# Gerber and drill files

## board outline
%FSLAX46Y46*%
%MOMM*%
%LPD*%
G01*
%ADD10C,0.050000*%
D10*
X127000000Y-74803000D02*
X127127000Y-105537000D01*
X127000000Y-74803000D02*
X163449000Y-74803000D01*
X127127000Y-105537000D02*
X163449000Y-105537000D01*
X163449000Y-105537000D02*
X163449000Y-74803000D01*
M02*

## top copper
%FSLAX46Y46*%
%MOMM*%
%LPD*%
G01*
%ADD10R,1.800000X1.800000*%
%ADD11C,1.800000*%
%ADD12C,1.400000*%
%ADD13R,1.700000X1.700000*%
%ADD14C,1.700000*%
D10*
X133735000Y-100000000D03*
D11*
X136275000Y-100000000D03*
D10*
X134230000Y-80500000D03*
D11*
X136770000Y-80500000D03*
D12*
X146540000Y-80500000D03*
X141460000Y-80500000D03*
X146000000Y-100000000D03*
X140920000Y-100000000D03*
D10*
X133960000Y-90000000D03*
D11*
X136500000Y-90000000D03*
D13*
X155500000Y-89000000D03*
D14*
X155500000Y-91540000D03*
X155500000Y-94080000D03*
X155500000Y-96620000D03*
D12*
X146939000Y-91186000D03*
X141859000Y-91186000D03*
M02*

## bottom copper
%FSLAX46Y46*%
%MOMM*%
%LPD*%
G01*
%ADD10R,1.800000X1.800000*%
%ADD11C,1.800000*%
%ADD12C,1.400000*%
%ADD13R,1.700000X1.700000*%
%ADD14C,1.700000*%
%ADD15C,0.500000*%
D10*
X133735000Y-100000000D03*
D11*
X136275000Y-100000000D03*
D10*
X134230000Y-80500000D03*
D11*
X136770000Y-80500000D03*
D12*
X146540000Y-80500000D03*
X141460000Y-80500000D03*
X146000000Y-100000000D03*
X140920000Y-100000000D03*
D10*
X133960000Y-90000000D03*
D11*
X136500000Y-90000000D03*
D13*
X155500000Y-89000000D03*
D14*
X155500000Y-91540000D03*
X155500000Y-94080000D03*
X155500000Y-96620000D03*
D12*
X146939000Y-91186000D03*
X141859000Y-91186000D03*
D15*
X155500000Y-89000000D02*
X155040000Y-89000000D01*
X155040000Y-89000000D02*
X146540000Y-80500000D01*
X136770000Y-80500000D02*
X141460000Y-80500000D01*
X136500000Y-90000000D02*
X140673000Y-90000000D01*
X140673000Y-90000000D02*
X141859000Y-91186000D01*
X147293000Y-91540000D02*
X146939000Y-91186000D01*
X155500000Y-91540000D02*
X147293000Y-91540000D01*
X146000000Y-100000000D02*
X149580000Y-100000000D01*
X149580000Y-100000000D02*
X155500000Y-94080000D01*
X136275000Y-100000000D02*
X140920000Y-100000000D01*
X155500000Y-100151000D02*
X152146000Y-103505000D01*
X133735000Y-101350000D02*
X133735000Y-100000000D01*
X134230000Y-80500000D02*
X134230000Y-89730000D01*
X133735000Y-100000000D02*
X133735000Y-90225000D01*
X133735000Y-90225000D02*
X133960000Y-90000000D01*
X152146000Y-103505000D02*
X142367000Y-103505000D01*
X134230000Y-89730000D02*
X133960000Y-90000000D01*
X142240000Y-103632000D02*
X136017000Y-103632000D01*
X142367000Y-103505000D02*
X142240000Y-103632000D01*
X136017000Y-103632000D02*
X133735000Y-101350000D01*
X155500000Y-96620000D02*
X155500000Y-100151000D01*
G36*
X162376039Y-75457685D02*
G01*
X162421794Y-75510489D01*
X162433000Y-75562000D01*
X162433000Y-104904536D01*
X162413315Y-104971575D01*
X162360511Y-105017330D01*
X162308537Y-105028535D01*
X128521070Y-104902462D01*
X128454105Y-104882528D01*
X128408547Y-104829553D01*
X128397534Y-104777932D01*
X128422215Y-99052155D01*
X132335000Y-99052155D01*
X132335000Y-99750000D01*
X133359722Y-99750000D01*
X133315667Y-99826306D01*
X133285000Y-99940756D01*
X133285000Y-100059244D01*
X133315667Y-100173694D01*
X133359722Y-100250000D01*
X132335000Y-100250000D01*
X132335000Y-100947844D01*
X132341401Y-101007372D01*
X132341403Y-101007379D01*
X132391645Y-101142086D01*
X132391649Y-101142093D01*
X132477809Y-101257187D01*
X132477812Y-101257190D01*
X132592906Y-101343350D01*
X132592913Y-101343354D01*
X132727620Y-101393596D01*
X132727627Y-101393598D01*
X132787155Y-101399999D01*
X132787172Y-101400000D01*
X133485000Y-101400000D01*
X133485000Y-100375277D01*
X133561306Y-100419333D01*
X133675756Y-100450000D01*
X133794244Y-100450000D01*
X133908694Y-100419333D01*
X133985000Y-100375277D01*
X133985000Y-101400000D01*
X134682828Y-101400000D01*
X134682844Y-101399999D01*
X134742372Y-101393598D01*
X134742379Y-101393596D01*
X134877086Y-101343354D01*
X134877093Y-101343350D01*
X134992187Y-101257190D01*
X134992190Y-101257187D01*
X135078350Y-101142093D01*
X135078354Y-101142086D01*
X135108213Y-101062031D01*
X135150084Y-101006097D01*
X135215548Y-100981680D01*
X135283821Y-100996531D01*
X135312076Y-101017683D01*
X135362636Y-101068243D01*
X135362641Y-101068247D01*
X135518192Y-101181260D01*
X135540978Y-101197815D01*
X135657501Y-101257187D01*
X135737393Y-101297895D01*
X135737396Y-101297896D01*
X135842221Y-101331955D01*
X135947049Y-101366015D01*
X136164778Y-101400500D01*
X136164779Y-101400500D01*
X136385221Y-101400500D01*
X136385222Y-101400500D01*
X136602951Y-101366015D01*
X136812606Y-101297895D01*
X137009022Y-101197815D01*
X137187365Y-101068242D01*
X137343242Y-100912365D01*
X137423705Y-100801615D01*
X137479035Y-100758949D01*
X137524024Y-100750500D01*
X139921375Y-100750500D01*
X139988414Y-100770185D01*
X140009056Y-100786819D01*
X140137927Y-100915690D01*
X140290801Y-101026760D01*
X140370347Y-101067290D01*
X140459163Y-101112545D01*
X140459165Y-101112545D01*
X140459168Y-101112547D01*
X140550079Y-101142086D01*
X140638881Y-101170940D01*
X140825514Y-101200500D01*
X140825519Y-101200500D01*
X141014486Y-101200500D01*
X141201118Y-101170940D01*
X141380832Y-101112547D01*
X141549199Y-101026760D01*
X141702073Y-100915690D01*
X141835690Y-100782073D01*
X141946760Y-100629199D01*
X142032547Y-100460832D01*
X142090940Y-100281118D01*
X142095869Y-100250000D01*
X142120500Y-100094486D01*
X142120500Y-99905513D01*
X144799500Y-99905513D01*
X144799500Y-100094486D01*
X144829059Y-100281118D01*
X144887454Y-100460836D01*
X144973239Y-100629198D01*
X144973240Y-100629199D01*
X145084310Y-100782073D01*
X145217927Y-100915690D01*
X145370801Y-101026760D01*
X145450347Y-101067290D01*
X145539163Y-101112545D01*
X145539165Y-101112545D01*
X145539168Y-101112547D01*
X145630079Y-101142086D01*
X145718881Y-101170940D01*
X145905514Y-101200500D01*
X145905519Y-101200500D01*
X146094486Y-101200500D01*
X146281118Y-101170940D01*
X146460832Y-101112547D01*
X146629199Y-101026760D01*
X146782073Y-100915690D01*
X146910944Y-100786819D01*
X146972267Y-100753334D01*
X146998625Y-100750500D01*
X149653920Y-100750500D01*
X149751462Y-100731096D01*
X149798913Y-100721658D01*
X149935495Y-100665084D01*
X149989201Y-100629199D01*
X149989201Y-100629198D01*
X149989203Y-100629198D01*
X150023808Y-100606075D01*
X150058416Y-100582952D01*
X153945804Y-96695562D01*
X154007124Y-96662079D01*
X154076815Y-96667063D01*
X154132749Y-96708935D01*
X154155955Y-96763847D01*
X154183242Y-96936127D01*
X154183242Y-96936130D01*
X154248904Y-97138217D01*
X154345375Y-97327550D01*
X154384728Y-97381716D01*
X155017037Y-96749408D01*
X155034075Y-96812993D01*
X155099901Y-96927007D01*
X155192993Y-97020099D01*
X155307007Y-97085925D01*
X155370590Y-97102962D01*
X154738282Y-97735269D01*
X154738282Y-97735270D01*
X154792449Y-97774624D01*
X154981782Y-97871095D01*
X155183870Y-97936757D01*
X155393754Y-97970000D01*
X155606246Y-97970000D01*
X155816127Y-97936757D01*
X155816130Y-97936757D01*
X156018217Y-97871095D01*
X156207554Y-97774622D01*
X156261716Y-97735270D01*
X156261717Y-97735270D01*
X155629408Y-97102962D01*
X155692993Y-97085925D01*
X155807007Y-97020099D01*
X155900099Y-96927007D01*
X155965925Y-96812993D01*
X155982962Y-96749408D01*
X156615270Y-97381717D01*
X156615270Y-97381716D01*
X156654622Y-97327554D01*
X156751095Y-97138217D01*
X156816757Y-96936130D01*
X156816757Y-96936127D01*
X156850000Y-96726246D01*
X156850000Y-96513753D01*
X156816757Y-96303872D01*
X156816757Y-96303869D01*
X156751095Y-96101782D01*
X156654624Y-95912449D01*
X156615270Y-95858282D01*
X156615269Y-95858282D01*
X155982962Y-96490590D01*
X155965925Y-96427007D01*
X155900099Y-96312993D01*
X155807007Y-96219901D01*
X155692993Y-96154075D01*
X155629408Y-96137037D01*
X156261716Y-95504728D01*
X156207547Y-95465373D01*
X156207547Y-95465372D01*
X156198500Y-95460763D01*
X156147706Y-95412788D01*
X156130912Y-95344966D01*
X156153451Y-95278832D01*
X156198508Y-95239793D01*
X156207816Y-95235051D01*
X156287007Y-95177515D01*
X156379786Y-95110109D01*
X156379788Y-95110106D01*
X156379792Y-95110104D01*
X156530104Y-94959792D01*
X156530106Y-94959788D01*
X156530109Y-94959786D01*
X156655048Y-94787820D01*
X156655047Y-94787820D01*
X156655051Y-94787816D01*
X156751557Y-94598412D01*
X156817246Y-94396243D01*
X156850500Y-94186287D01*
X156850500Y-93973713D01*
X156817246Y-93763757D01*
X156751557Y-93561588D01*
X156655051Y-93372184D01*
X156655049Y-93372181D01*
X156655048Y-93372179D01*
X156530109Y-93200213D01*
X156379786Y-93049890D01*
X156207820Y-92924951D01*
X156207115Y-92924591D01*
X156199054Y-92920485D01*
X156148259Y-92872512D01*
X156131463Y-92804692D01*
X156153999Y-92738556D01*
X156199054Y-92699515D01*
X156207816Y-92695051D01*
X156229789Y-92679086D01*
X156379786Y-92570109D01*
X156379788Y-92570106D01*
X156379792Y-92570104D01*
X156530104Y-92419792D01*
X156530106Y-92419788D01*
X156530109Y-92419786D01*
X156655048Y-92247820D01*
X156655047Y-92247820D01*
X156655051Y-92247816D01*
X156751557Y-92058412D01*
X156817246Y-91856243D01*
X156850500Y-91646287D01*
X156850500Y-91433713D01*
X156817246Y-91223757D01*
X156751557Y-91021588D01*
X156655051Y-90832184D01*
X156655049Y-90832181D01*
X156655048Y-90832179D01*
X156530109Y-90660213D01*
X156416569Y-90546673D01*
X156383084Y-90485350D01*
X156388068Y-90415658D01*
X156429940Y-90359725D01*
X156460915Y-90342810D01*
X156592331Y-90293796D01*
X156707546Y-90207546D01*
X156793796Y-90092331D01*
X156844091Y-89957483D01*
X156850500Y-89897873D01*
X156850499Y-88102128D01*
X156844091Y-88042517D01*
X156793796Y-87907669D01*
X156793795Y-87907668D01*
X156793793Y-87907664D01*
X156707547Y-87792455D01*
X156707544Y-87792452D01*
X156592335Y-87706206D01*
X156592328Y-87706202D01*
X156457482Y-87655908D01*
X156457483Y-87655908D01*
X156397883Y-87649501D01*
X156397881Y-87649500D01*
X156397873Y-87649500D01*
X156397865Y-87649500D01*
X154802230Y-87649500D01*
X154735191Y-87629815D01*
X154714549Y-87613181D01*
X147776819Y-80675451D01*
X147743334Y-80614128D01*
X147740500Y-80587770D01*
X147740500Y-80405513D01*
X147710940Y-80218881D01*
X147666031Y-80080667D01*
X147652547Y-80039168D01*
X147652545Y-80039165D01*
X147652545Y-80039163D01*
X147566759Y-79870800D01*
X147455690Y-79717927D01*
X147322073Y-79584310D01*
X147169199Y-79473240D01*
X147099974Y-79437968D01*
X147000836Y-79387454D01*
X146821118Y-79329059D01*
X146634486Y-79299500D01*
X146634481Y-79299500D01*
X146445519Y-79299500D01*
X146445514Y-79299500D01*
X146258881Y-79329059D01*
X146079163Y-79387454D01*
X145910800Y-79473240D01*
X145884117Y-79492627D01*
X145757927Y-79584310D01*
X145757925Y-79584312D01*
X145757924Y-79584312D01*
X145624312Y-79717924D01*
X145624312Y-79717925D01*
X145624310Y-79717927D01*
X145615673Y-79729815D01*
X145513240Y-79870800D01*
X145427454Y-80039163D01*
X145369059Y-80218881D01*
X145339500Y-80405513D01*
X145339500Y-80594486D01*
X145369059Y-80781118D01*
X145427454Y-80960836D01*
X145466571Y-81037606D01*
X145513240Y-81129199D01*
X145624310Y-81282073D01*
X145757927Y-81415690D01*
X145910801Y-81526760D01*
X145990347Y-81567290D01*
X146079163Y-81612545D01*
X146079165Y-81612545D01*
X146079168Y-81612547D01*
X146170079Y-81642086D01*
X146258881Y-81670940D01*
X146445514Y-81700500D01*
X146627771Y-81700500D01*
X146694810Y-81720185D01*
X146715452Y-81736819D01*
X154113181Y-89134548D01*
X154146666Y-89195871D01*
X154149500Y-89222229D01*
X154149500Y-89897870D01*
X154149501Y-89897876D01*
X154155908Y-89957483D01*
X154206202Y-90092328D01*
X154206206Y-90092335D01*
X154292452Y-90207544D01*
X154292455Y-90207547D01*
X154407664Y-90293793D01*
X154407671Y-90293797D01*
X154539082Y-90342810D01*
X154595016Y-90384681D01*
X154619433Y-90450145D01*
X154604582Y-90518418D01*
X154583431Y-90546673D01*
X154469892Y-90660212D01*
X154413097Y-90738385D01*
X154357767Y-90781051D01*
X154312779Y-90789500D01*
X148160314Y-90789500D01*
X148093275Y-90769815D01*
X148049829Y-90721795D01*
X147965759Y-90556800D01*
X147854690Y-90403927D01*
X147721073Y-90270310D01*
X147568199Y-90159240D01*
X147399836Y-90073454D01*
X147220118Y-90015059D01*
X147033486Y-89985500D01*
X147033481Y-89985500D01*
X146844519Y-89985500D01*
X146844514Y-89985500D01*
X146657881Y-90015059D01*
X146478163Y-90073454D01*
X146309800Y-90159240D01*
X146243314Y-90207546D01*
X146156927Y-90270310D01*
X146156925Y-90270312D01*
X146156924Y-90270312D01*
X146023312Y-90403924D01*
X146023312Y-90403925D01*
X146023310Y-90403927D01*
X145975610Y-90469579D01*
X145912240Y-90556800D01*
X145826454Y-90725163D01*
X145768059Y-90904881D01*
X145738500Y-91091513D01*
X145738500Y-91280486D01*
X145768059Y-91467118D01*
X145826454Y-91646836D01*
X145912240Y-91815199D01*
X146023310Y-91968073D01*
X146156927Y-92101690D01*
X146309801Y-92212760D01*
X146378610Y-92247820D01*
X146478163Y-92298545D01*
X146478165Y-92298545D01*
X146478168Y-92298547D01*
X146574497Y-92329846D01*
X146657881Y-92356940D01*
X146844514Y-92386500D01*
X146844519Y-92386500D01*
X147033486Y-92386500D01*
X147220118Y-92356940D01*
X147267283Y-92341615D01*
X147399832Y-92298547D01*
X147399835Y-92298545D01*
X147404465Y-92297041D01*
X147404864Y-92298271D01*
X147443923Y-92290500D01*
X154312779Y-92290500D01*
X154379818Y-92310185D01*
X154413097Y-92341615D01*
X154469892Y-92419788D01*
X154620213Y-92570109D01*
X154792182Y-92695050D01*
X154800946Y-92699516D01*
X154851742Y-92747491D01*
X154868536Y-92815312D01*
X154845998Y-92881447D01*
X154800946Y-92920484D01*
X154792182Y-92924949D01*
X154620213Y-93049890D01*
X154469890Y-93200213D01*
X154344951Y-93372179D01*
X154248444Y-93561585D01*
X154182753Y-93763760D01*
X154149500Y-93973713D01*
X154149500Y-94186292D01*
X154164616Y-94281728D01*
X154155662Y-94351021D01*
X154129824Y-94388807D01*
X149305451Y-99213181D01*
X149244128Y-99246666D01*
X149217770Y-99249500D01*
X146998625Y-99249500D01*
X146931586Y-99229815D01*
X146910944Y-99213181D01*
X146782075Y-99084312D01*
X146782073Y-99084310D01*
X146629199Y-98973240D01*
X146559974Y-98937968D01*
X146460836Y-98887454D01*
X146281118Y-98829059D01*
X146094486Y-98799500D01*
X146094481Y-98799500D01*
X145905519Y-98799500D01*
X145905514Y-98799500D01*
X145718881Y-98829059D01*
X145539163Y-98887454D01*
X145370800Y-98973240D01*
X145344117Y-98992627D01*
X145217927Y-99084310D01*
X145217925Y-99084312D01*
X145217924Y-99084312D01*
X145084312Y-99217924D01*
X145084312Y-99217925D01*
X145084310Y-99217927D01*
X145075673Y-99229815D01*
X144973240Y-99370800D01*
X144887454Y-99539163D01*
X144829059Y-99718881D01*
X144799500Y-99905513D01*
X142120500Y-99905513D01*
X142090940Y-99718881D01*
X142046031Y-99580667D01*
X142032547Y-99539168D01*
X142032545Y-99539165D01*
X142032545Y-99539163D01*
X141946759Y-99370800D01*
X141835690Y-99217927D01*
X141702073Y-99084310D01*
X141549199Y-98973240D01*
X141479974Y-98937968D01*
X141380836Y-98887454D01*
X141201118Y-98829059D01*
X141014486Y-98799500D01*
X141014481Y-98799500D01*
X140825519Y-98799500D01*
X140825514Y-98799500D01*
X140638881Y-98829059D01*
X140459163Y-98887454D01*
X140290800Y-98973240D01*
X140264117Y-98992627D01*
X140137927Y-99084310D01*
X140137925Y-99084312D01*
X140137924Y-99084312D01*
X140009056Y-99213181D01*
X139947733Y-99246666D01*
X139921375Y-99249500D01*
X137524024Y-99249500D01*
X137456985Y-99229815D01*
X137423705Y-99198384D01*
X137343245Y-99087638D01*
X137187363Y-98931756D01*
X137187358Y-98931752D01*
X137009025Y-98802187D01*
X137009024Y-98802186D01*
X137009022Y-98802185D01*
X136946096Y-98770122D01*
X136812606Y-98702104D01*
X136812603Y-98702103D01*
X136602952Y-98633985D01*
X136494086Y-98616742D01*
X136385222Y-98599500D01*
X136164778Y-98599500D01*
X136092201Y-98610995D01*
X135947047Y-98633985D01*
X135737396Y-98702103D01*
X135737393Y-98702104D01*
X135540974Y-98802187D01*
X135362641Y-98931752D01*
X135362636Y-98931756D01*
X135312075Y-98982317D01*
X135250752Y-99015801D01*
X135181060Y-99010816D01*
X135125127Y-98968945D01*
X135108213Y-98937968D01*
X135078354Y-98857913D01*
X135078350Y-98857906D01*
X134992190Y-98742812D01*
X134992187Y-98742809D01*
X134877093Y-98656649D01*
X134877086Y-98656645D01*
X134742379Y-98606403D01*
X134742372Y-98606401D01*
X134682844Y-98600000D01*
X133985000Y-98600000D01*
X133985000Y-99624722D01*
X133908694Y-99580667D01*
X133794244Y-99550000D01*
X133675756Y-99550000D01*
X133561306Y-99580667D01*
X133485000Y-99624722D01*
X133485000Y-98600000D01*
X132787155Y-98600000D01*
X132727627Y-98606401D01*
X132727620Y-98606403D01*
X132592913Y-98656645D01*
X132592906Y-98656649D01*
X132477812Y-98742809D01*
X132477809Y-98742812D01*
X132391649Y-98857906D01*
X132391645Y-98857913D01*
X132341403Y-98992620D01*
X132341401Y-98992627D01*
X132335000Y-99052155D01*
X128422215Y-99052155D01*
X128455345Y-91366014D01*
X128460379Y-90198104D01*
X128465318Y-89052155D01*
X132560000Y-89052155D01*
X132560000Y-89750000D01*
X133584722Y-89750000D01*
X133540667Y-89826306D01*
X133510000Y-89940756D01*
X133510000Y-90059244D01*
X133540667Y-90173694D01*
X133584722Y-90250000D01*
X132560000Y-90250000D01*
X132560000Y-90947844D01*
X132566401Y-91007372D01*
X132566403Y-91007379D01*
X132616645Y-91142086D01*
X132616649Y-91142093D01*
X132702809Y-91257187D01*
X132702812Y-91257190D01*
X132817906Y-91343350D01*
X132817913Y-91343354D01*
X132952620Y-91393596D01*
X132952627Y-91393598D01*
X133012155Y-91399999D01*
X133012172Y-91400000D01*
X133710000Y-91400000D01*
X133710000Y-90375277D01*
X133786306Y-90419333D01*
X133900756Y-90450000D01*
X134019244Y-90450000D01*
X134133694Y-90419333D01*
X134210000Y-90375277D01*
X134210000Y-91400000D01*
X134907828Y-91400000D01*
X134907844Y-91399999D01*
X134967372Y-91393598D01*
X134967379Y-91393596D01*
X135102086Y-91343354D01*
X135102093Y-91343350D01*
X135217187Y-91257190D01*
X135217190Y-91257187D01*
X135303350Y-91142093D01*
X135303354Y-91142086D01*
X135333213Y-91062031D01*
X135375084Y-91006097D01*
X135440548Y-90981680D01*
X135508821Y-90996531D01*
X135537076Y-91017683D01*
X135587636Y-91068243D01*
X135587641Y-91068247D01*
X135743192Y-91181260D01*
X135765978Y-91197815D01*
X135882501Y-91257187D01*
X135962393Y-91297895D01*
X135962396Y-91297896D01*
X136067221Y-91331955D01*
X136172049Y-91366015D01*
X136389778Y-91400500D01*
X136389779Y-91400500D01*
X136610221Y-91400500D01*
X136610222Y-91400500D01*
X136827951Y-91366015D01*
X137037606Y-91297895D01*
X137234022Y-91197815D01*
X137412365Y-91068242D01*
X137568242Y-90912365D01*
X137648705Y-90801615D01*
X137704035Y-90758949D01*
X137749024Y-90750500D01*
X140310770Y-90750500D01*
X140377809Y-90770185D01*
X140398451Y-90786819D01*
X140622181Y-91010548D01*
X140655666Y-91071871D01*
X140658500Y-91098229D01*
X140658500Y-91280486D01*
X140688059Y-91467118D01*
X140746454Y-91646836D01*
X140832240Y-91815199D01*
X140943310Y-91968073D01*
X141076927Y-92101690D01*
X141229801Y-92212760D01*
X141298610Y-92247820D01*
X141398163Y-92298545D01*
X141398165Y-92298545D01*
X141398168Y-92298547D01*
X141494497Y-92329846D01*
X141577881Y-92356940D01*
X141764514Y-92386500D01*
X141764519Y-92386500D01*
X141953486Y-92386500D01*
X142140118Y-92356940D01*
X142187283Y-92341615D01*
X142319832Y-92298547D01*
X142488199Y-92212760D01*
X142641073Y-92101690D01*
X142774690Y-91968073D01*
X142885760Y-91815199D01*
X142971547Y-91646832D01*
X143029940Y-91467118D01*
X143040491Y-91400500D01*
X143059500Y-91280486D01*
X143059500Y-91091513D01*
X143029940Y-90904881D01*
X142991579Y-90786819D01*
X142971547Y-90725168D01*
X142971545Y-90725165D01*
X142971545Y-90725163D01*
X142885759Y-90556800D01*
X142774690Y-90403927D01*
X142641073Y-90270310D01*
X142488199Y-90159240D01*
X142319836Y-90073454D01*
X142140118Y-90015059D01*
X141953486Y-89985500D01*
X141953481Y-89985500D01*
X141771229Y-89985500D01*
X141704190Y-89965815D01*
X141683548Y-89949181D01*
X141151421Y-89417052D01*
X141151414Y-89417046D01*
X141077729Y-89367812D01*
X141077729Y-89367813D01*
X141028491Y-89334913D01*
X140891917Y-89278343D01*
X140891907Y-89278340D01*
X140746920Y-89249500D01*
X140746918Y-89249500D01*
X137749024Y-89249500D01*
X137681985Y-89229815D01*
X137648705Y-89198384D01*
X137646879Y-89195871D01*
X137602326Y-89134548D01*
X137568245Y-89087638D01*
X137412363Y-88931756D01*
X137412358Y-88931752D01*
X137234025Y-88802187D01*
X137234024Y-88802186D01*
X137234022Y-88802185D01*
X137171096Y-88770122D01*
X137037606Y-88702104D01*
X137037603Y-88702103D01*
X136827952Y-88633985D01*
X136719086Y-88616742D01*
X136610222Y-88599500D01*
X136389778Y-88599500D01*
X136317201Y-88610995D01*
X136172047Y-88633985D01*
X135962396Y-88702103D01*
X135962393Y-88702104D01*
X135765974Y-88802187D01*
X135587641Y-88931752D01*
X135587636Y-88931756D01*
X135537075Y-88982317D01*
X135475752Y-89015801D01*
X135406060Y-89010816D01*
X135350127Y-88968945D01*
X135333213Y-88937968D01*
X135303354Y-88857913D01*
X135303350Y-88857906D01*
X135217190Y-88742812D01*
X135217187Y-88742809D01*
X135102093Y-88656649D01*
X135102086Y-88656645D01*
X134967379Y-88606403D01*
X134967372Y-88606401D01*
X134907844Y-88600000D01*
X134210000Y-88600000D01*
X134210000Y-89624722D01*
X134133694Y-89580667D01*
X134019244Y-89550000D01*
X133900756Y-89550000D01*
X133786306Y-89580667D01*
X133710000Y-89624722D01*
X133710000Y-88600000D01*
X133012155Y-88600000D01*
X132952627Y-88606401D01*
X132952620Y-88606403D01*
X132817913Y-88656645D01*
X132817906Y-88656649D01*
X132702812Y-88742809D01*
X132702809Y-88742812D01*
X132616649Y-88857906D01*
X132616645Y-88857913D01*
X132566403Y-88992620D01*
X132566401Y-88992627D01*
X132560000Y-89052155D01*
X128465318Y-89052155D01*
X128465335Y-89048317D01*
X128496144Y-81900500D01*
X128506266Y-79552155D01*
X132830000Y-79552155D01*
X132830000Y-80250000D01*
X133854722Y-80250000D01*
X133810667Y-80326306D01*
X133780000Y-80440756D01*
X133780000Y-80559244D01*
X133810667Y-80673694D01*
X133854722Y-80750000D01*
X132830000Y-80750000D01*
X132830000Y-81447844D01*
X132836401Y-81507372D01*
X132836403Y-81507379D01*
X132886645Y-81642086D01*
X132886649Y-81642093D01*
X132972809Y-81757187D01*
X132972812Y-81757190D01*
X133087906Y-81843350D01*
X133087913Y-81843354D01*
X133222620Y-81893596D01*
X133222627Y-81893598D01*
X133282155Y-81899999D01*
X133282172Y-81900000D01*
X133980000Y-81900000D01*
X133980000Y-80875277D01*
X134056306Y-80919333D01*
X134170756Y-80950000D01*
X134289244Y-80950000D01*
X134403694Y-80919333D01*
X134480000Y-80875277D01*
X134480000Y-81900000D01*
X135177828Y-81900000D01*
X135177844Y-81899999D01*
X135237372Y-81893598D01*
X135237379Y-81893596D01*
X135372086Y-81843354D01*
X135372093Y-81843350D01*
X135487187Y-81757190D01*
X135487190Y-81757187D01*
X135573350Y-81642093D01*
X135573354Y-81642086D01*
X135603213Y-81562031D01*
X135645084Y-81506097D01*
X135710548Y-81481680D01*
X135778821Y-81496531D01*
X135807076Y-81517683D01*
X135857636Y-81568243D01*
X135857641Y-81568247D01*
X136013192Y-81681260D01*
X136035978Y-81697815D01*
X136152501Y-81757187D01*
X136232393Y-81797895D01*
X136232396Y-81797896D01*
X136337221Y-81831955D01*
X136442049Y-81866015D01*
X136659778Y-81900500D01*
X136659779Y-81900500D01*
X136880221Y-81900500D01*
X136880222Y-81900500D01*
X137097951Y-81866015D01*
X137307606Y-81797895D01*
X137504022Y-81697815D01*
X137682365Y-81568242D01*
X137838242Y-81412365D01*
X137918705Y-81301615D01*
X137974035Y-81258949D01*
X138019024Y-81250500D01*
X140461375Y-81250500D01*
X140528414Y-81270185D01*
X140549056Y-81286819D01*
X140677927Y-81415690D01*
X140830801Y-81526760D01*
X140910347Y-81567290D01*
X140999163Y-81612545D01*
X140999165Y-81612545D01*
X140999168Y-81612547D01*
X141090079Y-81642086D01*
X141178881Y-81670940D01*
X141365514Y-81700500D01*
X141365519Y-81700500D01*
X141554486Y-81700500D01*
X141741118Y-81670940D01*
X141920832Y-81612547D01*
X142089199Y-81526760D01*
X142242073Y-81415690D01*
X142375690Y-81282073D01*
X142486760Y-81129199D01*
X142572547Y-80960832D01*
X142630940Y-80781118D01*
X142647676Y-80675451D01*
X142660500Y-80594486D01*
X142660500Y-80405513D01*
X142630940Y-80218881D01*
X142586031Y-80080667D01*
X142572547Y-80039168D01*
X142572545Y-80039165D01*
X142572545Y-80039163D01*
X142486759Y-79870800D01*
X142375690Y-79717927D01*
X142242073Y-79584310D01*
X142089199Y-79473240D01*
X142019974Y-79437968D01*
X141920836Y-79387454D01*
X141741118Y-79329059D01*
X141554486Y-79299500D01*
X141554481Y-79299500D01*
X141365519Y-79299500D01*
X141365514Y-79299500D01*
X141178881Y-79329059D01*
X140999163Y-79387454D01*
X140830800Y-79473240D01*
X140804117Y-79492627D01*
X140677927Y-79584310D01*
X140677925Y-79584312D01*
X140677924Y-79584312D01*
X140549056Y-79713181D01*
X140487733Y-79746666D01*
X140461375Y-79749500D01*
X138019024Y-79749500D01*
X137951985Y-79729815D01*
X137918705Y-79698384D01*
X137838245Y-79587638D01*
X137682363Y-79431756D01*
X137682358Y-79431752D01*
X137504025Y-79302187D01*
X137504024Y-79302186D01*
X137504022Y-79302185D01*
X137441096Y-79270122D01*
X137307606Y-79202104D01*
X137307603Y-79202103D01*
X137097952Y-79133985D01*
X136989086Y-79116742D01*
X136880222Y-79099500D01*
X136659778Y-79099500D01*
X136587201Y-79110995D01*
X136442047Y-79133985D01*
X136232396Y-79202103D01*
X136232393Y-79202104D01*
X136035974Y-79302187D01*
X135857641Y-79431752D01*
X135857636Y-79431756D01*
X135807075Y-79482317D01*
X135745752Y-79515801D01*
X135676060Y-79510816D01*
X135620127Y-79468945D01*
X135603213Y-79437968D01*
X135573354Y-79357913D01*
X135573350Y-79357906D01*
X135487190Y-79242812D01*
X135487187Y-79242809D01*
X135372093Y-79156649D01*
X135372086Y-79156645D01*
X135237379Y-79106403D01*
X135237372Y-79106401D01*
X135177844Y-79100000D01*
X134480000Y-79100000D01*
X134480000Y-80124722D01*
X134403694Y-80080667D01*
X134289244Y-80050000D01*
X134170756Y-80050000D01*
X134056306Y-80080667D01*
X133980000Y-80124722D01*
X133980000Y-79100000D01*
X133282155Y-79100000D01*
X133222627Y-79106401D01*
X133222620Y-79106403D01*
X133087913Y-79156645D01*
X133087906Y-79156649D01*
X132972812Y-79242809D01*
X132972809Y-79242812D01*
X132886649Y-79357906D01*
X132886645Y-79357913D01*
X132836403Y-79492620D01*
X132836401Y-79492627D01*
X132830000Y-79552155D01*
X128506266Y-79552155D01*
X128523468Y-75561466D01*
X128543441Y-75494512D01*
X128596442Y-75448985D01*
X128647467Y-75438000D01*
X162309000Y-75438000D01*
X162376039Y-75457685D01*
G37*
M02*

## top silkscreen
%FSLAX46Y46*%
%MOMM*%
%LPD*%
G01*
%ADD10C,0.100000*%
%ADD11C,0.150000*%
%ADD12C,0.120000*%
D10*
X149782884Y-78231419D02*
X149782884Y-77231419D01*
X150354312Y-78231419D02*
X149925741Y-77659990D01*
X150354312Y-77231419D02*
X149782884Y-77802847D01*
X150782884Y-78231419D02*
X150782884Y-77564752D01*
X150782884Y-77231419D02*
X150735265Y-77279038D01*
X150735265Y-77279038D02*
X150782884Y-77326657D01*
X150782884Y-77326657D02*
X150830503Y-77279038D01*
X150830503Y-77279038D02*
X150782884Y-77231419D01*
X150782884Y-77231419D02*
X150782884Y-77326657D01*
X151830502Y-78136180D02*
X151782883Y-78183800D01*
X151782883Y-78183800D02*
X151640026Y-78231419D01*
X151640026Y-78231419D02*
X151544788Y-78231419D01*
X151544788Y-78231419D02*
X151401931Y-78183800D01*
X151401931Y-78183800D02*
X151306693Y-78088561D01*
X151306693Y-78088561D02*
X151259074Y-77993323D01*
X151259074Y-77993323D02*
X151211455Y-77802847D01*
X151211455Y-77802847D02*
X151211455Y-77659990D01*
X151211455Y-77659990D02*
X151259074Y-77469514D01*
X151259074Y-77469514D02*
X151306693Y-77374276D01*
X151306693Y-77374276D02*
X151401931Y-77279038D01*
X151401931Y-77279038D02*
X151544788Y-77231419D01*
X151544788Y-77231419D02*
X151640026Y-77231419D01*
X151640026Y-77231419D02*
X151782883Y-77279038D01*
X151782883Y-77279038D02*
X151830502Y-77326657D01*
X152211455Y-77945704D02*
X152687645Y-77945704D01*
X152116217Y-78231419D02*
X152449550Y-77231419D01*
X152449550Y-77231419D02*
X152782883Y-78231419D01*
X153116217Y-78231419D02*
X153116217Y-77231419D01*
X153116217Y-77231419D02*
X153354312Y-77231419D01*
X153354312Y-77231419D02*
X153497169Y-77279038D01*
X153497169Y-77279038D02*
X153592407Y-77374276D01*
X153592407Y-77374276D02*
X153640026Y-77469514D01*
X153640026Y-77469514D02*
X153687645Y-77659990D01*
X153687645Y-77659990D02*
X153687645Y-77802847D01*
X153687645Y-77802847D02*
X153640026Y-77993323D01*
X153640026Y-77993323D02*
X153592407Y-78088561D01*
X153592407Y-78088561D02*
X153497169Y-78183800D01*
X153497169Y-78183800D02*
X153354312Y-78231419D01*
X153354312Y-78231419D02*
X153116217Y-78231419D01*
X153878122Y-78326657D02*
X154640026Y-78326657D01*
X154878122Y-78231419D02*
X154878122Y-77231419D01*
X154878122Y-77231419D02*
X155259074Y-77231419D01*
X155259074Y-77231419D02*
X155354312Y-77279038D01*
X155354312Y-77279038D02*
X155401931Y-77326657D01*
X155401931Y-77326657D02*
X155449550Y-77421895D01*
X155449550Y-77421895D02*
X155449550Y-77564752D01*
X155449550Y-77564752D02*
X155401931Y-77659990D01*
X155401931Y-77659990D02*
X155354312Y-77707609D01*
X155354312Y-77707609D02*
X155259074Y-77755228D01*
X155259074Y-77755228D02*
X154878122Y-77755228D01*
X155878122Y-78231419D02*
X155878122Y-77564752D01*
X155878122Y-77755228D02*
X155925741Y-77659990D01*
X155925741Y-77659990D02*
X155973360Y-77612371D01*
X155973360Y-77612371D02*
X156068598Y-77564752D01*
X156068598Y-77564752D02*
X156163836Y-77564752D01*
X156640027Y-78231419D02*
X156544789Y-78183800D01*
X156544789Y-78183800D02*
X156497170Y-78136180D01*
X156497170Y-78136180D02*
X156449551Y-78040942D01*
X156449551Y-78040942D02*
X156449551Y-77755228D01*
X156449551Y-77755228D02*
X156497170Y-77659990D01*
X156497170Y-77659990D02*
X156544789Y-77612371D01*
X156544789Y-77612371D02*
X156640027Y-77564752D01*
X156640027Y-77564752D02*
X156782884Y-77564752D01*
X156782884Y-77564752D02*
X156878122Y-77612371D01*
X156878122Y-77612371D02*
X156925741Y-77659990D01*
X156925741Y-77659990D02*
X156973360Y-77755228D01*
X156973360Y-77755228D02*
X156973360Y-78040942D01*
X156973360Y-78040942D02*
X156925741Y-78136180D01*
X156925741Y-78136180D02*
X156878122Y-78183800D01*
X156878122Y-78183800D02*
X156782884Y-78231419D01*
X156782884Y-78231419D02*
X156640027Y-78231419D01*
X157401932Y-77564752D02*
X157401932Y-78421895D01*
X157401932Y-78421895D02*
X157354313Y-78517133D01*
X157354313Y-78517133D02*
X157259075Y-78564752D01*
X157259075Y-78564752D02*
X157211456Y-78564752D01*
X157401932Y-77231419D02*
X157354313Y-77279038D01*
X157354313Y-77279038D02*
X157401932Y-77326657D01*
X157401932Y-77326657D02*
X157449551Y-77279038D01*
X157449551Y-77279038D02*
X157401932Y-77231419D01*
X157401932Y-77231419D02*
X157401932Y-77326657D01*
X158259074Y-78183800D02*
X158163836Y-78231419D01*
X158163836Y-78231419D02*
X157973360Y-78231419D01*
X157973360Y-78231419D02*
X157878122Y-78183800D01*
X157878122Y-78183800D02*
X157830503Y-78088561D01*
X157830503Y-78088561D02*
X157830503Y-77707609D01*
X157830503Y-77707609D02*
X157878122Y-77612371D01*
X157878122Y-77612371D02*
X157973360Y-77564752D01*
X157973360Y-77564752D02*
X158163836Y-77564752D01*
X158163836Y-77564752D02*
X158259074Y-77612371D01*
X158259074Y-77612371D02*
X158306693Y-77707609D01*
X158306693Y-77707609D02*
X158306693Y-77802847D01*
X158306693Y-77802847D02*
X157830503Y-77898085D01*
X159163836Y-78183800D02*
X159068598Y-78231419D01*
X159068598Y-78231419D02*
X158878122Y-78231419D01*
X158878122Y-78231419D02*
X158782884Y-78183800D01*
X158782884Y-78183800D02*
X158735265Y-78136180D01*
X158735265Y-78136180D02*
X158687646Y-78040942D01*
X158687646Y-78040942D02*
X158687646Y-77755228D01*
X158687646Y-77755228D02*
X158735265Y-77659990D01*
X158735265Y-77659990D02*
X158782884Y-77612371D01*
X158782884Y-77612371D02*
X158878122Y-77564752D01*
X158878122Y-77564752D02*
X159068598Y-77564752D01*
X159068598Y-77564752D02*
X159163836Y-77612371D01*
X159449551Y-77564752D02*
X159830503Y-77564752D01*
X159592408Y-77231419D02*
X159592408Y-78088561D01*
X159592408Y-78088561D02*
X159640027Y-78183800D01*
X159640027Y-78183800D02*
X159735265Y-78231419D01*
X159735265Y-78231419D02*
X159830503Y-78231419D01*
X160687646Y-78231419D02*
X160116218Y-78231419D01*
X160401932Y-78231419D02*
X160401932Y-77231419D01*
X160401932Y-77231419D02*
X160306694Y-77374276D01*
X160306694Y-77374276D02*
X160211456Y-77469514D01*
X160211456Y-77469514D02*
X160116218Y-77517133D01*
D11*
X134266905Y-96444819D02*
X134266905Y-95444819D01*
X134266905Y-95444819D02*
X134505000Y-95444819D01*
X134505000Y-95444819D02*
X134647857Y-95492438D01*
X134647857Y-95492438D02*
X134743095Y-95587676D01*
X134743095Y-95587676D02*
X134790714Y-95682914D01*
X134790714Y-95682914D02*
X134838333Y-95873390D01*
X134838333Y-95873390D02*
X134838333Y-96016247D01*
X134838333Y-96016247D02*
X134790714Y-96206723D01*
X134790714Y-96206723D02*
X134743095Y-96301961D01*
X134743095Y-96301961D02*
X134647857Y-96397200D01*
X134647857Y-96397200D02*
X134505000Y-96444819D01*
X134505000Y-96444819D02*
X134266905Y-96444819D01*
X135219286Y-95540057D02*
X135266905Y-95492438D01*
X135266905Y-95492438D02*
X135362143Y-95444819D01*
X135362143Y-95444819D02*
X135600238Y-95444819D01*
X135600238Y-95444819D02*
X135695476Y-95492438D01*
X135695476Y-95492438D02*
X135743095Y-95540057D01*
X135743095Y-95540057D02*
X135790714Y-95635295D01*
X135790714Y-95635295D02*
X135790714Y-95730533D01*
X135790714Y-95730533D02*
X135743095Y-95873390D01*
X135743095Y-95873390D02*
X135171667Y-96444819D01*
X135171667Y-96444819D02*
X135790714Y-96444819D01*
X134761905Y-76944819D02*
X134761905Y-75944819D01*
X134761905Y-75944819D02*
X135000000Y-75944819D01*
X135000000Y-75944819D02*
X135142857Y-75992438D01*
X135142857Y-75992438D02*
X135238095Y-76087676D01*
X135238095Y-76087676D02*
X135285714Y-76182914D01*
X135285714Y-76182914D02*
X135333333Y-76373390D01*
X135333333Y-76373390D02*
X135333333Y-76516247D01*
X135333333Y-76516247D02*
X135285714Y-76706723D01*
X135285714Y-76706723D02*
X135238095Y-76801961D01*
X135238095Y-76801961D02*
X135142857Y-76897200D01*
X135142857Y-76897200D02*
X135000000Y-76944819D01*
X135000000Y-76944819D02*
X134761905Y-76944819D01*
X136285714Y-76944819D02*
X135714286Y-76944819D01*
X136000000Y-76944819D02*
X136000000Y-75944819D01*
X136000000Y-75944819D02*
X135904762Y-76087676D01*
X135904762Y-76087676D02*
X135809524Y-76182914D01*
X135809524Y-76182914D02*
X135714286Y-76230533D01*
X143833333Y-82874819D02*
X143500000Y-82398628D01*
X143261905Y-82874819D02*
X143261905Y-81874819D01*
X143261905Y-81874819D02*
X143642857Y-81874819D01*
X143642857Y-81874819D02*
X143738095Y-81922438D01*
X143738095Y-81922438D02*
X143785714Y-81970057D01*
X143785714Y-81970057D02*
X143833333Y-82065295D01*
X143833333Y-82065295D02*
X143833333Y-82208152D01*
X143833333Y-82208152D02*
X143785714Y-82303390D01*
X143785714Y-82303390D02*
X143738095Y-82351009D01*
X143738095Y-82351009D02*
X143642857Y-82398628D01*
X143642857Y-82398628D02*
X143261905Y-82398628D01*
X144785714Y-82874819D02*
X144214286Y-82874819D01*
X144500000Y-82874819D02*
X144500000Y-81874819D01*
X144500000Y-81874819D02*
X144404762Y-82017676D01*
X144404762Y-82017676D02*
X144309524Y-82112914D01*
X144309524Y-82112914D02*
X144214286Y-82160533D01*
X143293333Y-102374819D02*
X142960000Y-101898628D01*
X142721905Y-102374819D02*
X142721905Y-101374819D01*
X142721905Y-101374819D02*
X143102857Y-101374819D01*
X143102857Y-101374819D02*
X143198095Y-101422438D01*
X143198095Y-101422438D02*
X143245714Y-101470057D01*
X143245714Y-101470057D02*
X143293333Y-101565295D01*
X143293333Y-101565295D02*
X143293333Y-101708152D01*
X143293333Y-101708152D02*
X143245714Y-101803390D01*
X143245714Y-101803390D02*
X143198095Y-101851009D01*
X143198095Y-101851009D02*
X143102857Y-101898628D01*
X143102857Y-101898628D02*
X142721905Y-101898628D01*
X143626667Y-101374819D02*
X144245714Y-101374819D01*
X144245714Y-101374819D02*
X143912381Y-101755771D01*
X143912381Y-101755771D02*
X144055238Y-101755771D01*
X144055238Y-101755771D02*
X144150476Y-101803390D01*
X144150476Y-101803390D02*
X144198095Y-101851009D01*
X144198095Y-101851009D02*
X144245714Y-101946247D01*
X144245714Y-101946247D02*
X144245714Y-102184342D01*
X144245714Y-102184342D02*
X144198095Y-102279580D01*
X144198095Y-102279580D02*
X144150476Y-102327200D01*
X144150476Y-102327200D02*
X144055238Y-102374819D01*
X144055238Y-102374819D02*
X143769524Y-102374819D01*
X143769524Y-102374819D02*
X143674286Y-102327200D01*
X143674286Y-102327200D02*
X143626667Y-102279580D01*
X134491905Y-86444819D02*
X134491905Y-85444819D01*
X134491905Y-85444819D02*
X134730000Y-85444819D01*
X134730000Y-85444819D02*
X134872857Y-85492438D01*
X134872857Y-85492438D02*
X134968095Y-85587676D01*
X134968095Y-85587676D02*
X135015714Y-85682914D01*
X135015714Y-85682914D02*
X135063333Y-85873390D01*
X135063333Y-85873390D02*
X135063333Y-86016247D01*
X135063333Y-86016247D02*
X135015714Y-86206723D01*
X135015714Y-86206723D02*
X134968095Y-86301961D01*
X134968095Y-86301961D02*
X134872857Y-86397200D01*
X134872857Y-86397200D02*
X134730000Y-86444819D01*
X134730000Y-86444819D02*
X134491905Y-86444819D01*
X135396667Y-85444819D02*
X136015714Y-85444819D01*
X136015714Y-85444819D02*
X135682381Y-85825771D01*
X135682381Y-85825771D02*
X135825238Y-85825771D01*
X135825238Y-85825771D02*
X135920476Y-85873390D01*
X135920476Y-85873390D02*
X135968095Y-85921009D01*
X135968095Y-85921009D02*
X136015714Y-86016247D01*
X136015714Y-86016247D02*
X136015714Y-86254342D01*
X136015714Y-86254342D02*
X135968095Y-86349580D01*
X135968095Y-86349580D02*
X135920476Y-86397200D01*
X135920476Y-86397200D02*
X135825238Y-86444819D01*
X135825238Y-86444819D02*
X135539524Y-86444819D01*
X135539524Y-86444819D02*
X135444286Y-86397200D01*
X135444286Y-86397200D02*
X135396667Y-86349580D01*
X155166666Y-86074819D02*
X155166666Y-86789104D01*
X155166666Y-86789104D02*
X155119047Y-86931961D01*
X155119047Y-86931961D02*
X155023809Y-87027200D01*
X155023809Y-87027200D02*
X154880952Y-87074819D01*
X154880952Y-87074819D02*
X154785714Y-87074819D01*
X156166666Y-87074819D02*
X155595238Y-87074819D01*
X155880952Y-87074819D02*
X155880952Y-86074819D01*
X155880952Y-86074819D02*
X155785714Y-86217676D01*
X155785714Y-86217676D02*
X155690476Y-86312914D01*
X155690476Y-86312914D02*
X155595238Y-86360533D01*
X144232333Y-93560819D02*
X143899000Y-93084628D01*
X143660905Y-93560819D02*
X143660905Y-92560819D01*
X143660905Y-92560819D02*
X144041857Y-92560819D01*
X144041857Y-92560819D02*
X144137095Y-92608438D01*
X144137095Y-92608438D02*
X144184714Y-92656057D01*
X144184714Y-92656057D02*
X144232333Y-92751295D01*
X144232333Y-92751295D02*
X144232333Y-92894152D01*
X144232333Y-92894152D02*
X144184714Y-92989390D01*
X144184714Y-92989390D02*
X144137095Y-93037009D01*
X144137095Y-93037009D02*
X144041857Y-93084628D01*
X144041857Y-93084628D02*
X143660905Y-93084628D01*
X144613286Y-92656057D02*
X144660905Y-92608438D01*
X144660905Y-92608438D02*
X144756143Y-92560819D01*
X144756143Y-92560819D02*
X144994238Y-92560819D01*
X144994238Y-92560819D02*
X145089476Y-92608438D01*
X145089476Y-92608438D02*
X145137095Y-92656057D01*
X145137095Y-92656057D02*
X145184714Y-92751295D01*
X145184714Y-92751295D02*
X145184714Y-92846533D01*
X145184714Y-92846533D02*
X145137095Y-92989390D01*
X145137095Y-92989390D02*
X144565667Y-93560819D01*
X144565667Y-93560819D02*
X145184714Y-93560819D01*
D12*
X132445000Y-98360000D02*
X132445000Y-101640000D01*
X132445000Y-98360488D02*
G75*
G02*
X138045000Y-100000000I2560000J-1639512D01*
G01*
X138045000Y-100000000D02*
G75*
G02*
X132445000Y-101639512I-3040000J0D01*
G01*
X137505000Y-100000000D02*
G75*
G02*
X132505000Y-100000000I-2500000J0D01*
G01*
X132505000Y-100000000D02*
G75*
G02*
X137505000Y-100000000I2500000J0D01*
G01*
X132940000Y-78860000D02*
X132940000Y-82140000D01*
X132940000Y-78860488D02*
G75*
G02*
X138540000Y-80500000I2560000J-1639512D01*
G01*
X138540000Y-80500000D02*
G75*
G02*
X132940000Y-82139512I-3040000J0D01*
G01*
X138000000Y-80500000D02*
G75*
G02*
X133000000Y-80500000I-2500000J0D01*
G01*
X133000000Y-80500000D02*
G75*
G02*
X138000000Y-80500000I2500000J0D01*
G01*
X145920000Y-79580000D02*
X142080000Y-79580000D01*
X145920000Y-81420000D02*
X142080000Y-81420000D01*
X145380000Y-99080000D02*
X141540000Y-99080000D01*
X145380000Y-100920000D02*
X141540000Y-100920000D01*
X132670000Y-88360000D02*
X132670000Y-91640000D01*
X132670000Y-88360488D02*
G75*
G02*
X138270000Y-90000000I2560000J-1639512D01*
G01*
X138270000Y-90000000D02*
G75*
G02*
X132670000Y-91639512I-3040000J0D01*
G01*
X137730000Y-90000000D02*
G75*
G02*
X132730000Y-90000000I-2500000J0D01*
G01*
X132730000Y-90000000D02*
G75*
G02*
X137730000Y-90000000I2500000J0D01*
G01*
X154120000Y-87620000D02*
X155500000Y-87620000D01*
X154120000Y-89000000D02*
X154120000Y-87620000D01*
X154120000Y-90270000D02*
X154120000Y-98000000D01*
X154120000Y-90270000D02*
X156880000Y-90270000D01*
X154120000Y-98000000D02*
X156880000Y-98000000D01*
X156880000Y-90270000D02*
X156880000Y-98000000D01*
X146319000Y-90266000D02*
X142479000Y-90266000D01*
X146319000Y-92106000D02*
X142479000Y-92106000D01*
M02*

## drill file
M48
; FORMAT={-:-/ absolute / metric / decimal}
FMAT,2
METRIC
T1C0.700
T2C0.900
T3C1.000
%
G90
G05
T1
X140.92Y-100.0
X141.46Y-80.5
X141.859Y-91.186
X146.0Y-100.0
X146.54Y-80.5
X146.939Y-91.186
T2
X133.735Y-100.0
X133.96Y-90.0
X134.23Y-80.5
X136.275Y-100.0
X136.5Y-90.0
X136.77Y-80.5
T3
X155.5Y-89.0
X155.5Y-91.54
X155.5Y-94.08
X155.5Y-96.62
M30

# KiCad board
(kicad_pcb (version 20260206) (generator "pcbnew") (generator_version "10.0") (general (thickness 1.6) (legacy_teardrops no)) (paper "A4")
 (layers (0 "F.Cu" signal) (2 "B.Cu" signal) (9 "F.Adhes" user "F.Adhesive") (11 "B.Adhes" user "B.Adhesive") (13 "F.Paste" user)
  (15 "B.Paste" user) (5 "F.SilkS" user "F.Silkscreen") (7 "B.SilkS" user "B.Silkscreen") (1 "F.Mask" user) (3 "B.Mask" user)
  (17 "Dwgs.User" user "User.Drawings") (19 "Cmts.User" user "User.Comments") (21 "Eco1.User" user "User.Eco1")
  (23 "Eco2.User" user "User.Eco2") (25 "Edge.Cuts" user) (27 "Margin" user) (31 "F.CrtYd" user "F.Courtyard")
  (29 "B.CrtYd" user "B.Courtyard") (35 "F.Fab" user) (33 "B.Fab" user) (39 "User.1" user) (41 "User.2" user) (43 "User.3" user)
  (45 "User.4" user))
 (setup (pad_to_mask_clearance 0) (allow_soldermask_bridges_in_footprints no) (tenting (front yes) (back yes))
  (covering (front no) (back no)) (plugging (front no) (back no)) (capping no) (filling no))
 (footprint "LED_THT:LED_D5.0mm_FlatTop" (layer "F.Cu") (at 133.735 100)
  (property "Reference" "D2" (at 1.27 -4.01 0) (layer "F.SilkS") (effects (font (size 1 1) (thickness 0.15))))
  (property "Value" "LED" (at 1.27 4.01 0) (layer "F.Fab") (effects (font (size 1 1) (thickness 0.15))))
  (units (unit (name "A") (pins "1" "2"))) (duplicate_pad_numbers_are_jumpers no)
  (fp_line (start -1.29 -1.64) (end -1.29 1.64) (stroke (width 0.12) (type solid)) (layer "F.SilkS"))
  (fp_arc (start -1.29 -1.639512) (mid 2.124166 -2.917533) (end 4.31 0) (stroke (width 0.12) (type solid)) (layer "F.SilkS"))
  (fp_arc (start 4.31 0) (mid 2.124166 2.917533) (end -1.29 1.639512) (stroke (width 0.12) (type solid)) (layer "F.SilkS"))
  (fp_circle (center 1.27 0) (end 3.77 0) (stroke (width 0.12) (type solid)) (fill no) (layer "F.SilkS"))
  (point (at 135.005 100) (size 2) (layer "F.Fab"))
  (pad "1" thru_hole rect (at 0 0) (size 1.8 1.8) (drill 0.9) (layers "*.Cu" "*.Mask") (remove_unused_layers no) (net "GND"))
  (pad "2" thru_hole circle (at 2.54 0) (size 1.8 1.8) (drill 0.9) (layers "*.Cu" "*.Mask") (remove_unused_layers no) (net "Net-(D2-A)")))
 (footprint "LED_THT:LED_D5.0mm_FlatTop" (layer "F.Cu") (at 134.23 80.5)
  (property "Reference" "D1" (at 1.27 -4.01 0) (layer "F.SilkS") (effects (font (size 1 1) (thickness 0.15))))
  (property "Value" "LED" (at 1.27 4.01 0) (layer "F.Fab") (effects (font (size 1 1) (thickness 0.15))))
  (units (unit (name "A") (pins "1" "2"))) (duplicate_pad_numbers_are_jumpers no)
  (fp_line (start -1.29 -1.64) (end -1.29 1.64) (stroke (width 0.12) (type solid)) (layer "F.SilkS"))
  (fp_arc (start -1.29 -1.639512) (mid 2.124166 -2.917533) (end 4.31 0) (stroke (width 0.12) (type solid)) (layer "F.SilkS"))
  (fp_arc (start 4.31 0) (mid 2.124166 2.917533) (end -1.29 1.639512) (stroke (width 0.12) (type solid)) (layer "F.SilkS"))
  (fp_circle (center 1.27 0) (end 3.77 0) (stroke (width 0.12) (type solid)) (fill no) (layer "F.SilkS"))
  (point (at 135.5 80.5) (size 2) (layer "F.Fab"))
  (pad "1" thru_hole rect (at 0 0) (size 1.8 1.8) (drill 0.9) (layers "*.Cu" "*.Mask") (remove_unused_layers no) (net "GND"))
  (pad "2" thru_hole circle (at 2.54 0) (size 1.8 1.8) (drill 0.9) (layers "*.Cu" "*.Mask") (remove_unused_layers no) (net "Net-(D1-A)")))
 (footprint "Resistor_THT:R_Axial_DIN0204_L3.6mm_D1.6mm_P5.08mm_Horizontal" (layer "F.Cu") (at 146.54 80.5 180)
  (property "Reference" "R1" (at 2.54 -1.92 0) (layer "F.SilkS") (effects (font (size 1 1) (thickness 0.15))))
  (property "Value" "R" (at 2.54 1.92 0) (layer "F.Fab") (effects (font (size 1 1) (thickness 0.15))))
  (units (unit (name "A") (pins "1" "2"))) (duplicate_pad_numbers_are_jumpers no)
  (fp_line (start 0.62 0.92) (end 4.46 0.92) (stroke (width 0.12) (type solid)) (layer "F.SilkS"))
  (fp_line (start 0.62 -0.92) (end 4.46 -0.92) (stroke (width 0.12) (type solid)) (layer "F.SilkS"))
  (pad "1" thru_hole circle (at 0 0 180) (size 1.4 1.4) (drill 0.7) (layers "*.Cu" "*.Mask") (remove_unused_layers no)
   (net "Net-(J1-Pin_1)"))
  (pad "2" thru_hole circle (at 5.08 0 180) (size 1.4 1.4) (drill 0.7) (layers "*.Cu" "*.Mask") (remove_unused_layers no) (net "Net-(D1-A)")))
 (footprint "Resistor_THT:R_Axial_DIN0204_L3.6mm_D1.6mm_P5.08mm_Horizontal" (layer "F.Cu") (at 146 100 180)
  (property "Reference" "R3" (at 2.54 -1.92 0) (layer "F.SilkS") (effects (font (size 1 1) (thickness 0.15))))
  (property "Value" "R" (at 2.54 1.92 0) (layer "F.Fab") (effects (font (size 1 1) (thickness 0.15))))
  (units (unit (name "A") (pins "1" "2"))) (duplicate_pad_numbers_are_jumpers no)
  (fp_line (start 0.62 0.92) (end 4.46 0.92) (stroke (width 0.12) (type solid)) (layer "F.SilkS"))
  (fp_line (start 0.62 -0.92) (end 4.46 -0.92) (stroke (width 0.12) (type solid)) (layer "F.SilkS"))
  (pad "1" thru_hole circle (at 0 0 180) (size 1.4 1.4) (drill 0.7) (layers "*.Cu" "*.Mask") (remove_unused_layers no)
   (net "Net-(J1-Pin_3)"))
  (pad "2" thru_hole circle (at 5.08 0 180) (size 1.4 1.4) (drill 0.7) (layers "*.Cu" "*.Mask") (remove_unused_layers no) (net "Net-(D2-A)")))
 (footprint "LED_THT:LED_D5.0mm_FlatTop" (layer "F.Cu") (at 133.96 90)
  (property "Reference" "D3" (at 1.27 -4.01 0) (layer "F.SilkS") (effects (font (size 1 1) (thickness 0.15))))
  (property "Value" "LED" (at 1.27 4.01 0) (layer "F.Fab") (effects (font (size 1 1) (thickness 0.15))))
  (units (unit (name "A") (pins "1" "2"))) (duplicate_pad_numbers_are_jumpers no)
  (fp_line (start -1.29 -1.64) (end -1.29 1.64) (stroke (width 0.12) (type solid)) (layer "F.SilkS"))
  (fp_arc (start -1.29 -1.639512) (mid 2.124166 -2.917533) (end 4.31 0) (stroke (width 0.12) (type solid)) (layer "F.SilkS"))
  (fp_arc (start 4.31 0) (mid 2.124166 2.917533) (end -1.29 1.639512) (stroke (width 0.12) (type solid)) (layer "F.SilkS"))
  (fp_circle (center 1.27 0) (end 3.77 0) (stroke (width 0.12) (type solid)) (fill no) (layer "F.SilkS"))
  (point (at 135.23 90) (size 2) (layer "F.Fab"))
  (pad "1" thru_hole rect (at 0 0) (size 1.8 1.8) (drill 0.9) (layers "*.Cu" "*.Mask") (remove_unused_layers no) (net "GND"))
  (pad "2" thru_hole circle (at 2.54 0) (size 1.8 1.8) (drill 0.9) (layers "*.Cu" "*.Mask") (remove_unused_layers no) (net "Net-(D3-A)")))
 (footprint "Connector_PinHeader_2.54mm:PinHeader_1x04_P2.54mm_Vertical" (layer "F.Cu") (at 155.5 89)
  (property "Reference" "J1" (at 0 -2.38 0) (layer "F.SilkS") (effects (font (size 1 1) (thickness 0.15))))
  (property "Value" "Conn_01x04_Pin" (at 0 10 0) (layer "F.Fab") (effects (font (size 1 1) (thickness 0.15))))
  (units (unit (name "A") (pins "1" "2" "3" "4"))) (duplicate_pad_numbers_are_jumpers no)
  (fp_line (start -1.38 -1.38) (end 0 -1.38) (stroke (width 0.12) (type solid)) (layer "F.SilkS"))
  (fp_line (start -1.38 0) (end -1.38 -1.38) (stroke (width 0.12) (type solid)) (layer "F.SilkS"))
  (fp_line (start -1.38 1.27) (end -1.38 9) (stroke (width 0.12) (type solid)) (layer "F.SilkS"))
  (fp_line (start -1.38 1.27) (end 1.38 1.27) (stroke (width 0.12) (type solid)) (layer "F.SilkS"))
  (fp_line (start -1.38 9) (end 1.38 9) (stroke (width 0.12) (type solid)) (layer "F.SilkS"))
  (fp_line (start 1.38 1.27) (end 1.38 9) (stroke (width 0.12) (type solid)) (layer "F.SilkS"))
  (pad "1" thru_hole rect (at 0 0) (size 1.7 1.7) (drill 1) (layers "*.Cu" "*.Mask") (remove_unused_layers no) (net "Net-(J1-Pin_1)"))
  (pad "2" thru_hole circle (at 0 2.54) (size 1.7 1.7) (drill 1) (layers "*.Cu" "*.Mask") (remove_unused_layers no) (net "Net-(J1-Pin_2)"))
  (pad "3" thru_hole circle (at 0 5.08) (size 1.7 1.7) (drill 1) (layers "*.Cu" "*.Mask") (remove_unused_layers no) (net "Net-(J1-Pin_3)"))
  (pad "4" thru_hole circle (at 0 7.62) (size 1.7 1.7) (drill 1) (layers "*.Cu" "*.Mask") (remove_unused_layers no) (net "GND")))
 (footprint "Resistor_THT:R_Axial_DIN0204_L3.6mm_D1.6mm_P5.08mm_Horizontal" (layer "F.Cu") (at 146.939 91.186 180)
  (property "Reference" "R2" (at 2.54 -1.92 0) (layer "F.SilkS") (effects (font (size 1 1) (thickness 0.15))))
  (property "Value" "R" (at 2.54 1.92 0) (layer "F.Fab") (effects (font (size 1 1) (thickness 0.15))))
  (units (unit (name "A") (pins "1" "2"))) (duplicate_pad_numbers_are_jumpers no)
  (fp_line (start 0.62 0.92) (end 4.46 0.92) (stroke (width 0.12) (type solid)) (layer "F.SilkS"))
  (fp_line (start 0.62 -0.92) (end 4.46 -0.92) (stroke (width 0.12) (type solid)) (layer "F.SilkS"))
  (pad "1" thru_hole circle (at 0 0 180) (size 1.4 1.4) (drill 0.7) (layers "*.Cu" "*.Mask") (remove_unused_layers no)
   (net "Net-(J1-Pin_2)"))
  (pad "2" thru_hole circle (at 5.08 0 180) (size 1.4 1.4) (drill 0.7) (layers "*.Cu" "*.Mask") (remove_unused_layers no) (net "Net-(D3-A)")))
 (gr_line (start 127 74.803) (end 127.127 105.537) (stroke (width 0.05) (type default)) (layer "Edge.Cuts"))
 (gr_line (start 127 74.803) (end 163.449 74.803) (stroke (width 0.05) (type default)) (layer "Edge.Cuts"))
 (gr_line (start 127.127 105.537) (end 163.449 105.537) (stroke (width 0.05) (type default)) (layer "Edge.Cuts"))
 (gr_line (start 163.449 105.537) (end 163.449 74.803) (stroke (width 0.05) (type default)) (layer "Edge.Cuts"))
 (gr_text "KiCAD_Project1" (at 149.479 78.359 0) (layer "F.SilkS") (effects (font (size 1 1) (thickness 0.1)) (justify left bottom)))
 (segment (start 155.5 89) (end 155.04 89) (width 0.5) (layer "B.Cu") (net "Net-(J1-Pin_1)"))
 (segment (start 155.04 89) (end 146.54 80.5) (width 0.5) (layer "B.Cu") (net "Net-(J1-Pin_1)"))
 (segment (start 136.77 80.5) (end 141.46 80.5) (width 0.5) (layer "B.Cu") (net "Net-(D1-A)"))
 (segment (start 136.5 90) (end 140.673 90) (width 0.5) (layer "B.Cu") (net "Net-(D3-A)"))
 (segment (start 140.673 90) (end 141.859 91.186) (width 0.5) (layer "B.Cu") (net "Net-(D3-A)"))
 (segment (start 147.293 91.54) (end 146.939 91.186) (width 0.5) (layer "B.Cu") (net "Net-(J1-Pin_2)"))
 (segment (start 155.5 91.54) (end 147.293 91.54) (width 0.5) (layer "B.Cu") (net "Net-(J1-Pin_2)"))
 (segment (start 146 100) (end 149.58 100) (width 0.5) (layer "B.Cu") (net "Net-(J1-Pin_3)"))
 (segment (start 149.58 100) (end 155.5 94.08) (width 0.5) (layer "B.Cu") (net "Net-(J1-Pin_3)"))
 (segment (start 136.275 100) (end 140.92 100) (width 0.5) (layer "B.Cu") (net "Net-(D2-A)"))
 (segment (start 155.5 100.151) (end 152.146 103.505) (width 0.5) (layer "B.Cu") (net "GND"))
 (segment (start 133.735 101.35) (end 133.735 100) (width 0.5) (layer "B.Cu") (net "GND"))
 (segment (start 134.23 80.5) (end 134.23 89.73) (width 0.5) (layer "B.Cu") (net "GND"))
 (segment (start 133.735 100) (end 133.735 90.225) (width 0.5) (layer "B.Cu") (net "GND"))
 (segment (start 133.735 90.225) (end 133.96 90) (width 0.5) (layer "B.Cu") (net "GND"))
 (segment (start 152.146 103.505) (end 142.367 103.505) (width 0.5) (layer "B.Cu") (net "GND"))
 (segment (start 134.23 89.73) (end 133.96 90) (width 0.5) (layer "B.Cu") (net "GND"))
 (segment (start 142.24 103.632) (end 136.017 103.632) (width 0.5) (layer "B.Cu") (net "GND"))
 (segment (start 142.367 103.505) (end 142.24 103.632) (width 0.5) (layer "B.Cu") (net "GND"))
 (segment (start 136.017 103.632) (end 133.735 101.35) (width 0.5) (layer "B.Cu") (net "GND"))
 (segment (start 155.5 96.62) (end 155.5 100.151) (width 0.5) (layer "B.Cu") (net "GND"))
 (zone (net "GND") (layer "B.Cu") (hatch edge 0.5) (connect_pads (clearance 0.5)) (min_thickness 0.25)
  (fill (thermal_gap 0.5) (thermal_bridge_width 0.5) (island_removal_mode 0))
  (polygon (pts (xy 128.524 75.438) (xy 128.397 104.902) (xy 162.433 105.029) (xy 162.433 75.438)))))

